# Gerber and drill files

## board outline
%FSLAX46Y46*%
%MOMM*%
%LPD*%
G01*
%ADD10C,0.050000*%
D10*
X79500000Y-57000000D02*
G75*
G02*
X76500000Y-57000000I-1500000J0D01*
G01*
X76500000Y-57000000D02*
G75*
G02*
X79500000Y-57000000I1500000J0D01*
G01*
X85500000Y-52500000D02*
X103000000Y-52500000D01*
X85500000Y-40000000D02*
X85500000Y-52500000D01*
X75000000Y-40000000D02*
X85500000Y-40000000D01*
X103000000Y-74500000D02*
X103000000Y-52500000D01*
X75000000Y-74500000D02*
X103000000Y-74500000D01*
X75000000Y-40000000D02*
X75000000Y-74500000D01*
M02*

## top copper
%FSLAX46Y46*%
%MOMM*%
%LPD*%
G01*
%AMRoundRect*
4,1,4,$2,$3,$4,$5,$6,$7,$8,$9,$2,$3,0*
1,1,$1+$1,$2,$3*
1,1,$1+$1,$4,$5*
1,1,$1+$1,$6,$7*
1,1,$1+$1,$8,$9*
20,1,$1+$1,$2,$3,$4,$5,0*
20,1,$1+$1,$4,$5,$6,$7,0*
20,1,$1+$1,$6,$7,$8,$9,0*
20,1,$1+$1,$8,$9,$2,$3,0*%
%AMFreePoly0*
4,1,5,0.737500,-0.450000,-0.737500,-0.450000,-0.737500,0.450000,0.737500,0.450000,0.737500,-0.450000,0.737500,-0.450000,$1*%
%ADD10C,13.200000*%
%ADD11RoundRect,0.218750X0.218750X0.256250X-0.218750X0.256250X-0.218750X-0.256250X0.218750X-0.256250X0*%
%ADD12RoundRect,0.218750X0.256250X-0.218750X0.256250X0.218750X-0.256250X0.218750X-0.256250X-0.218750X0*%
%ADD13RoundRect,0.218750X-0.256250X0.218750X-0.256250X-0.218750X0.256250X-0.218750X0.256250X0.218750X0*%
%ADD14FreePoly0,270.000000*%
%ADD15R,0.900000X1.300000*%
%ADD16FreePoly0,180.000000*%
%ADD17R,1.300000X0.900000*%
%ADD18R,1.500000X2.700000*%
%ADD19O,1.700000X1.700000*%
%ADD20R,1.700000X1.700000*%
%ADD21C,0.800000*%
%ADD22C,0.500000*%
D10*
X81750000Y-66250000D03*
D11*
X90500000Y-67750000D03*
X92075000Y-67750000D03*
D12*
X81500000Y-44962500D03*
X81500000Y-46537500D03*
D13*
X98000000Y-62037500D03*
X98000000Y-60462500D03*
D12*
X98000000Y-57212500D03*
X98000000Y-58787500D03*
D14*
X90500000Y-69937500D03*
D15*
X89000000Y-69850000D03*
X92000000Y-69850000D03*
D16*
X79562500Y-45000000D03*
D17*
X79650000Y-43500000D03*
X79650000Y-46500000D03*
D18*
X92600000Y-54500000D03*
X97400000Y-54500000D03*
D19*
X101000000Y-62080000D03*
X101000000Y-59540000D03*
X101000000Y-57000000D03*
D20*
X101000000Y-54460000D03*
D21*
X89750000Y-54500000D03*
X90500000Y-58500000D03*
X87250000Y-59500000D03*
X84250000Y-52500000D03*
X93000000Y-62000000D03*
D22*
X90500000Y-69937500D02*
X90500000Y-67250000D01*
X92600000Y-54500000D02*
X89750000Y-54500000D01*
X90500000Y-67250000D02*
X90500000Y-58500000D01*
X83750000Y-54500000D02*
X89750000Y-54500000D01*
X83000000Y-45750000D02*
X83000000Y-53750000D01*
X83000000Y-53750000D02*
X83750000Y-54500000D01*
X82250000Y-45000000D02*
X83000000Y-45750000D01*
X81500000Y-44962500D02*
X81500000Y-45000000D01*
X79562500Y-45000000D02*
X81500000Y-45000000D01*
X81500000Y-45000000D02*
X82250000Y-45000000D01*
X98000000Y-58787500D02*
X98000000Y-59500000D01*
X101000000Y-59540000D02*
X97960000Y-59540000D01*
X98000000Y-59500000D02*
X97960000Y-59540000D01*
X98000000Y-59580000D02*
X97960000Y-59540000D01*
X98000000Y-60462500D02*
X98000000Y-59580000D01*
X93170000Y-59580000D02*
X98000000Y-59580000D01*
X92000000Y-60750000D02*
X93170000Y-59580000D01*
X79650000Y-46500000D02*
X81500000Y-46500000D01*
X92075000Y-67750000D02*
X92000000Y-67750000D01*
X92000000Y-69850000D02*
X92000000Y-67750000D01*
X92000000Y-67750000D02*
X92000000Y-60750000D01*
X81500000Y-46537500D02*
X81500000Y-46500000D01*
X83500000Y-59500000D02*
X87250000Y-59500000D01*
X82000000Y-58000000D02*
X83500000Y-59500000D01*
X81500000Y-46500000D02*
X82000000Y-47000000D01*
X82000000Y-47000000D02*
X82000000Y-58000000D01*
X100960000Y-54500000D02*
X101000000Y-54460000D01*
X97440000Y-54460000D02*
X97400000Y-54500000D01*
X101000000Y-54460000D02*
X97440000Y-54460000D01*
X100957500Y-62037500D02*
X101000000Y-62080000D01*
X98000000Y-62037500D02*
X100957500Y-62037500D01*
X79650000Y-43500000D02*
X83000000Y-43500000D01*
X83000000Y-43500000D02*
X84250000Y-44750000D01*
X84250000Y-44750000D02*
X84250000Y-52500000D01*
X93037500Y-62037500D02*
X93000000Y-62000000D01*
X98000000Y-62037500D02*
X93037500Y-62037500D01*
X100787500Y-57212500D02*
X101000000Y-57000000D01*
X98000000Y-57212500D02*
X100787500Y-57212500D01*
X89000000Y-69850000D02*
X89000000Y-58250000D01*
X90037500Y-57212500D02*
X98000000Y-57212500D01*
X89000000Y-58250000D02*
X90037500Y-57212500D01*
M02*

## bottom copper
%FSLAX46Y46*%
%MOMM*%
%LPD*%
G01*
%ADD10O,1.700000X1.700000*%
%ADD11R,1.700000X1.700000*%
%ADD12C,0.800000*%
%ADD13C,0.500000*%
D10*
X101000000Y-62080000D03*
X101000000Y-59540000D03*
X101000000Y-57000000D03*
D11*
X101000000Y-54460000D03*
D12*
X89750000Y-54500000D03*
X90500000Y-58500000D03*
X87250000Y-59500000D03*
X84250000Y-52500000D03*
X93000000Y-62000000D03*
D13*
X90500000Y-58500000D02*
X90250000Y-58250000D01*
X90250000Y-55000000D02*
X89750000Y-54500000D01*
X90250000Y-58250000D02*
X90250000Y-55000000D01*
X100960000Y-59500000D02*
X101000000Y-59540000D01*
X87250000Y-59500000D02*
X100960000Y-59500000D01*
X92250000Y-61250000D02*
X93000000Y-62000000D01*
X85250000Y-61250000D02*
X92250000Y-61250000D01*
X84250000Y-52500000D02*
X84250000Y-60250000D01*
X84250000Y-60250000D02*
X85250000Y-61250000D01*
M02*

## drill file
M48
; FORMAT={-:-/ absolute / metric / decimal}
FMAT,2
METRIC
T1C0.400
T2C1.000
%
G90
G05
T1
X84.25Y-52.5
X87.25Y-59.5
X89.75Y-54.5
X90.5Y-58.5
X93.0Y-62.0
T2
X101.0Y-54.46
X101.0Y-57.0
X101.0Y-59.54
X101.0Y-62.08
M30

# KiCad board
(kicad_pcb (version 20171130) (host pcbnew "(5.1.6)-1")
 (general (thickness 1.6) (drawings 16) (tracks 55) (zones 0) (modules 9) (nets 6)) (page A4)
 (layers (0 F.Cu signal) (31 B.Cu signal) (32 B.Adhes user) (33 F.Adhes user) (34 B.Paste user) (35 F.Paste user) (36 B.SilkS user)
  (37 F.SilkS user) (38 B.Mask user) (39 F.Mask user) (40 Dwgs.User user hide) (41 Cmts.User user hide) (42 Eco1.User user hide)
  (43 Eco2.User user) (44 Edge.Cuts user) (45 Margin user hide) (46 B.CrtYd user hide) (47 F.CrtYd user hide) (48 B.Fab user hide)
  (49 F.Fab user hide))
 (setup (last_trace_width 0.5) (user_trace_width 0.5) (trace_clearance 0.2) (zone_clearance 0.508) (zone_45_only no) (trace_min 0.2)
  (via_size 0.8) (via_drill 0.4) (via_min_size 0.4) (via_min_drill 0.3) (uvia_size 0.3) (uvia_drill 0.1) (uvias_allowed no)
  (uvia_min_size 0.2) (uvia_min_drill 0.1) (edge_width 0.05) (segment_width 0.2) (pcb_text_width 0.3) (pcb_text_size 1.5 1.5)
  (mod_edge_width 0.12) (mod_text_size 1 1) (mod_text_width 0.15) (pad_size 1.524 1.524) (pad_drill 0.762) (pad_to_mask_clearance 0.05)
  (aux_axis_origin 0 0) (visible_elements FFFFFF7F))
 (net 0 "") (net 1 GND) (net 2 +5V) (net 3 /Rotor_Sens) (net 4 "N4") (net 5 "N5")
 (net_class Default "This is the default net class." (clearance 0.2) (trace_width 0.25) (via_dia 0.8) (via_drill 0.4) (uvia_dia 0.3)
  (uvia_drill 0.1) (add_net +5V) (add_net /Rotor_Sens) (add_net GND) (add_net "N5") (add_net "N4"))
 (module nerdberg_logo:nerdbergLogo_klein (layer F.Cu) (at 81.8 66.25)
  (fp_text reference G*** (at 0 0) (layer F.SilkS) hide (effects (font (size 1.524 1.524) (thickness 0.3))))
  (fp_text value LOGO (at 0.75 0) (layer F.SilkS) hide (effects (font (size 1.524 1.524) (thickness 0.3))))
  (pad e1 smd circle (at -0.05 0) (size 13.2 13.2) (layers F.Cu)))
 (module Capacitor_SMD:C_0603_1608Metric (layer F.Cu) (at 91.2875 67.75 180)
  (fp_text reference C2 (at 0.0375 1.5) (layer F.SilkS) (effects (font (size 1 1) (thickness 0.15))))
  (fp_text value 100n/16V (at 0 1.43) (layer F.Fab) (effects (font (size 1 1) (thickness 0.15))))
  (pad 2 smd roundrect (at 0.7875 0 180) (size 0.875 0.95) (layers F.Cu F.Paste F.Mask) (roundrect_rratio 0.25) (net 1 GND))
  (pad 1 smd roundrect (at -0.7875 0 180) (size 0.875 0.95) (layers F.Cu F.Paste F.Mask) (roundrect_rratio 0.25) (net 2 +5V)))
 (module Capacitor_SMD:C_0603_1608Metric (layer F.Cu) (at 81.5 45.75 90)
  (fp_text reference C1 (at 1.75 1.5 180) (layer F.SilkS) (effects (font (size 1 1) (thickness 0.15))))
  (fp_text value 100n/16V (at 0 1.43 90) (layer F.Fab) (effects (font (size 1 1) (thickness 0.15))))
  (pad 2 smd roundrect (at 0.7875 0 90) (size 0.875 0.95) (layers F.Cu F.Paste F.Mask) (roundrect_rratio 0.25) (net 1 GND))
  (pad 1 smd roundrect (at -0.7875 0 90) (size 0.875 0.95) (layers F.Cu F.Paste F.Mask) (roundrect_rratio 0.25) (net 2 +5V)))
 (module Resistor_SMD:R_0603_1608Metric (layer F.Cu) (at 98 61.25 270)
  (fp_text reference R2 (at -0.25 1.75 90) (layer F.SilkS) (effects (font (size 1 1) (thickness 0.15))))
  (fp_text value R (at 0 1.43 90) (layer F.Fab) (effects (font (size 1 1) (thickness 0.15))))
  (pad 2 smd roundrect (at 0.7875 0 270) (size 0.875 0.95) (layers F.Cu F.Paste F.Mask) (roundrect_rratio 0.25) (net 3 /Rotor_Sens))
  (pad 1 smd roundrect (at -0.7875 0 270) (size 0.875 0.95) (layers F.Cu F.Paste F.Mask) (roundrect_rratio 0.25) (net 2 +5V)))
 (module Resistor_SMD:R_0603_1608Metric (layer F.Cu) (at 98 58 90)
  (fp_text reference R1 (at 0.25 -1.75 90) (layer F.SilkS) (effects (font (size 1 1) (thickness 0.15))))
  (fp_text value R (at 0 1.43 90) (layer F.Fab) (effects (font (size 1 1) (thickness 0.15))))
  (pad 2 smd roundrect (at 0.7875 0 90) (size 0.875 0.95) (layers F.Cu F.Paste F.Mask) (roundrect_rratio 0.25) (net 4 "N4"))
  (pad 1 smd roundrect (at -0.7875 0 90) (size 0.875 0.95) (layers F.Cu F.Paste F.Mask) (roundrect_rratio 0.25) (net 2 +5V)))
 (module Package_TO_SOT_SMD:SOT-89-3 (layer F.Cu) (at 90.5 71.5 270)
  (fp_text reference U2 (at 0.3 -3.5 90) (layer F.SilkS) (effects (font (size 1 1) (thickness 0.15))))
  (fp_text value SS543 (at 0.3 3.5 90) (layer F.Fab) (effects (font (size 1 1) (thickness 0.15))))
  (pad 2 smd custom (at -1.5625 0 270) (size 1.475 0.9) (layers F.Cu F.Paste F.Mask) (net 1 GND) (zone_connect 2)
   (options (clearance outline) (anchor rect)) (primitives))
  (pad 3 smd rect (at -1.65 1.5 270) (size 1.3 0.9) (layers F.Cu F.Paste F.Mask) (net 4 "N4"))
  (pad 1 smd rect (at -1.65 -1.5 270) (size 1.3 0.9) (layers F.Cu F.Paste F.Mask) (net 2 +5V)))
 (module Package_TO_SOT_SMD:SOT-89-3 (layer F.Cu) (at 78 45 180)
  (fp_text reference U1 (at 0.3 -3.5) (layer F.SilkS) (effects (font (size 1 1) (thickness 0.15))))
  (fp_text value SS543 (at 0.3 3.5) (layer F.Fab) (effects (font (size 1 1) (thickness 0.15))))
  (pad 2 smd custom (at -1.5625 0 180) (size 1.475 0.9) (layers F.Cu F.Paste F.Mask) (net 1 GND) (zone_connect 2)
   (options (clearance outline) (anchor rect)) (primitives))
  (pad 3 smd rect (at -1.65 1.5 180) (size 1.3 0.9) (layers F.Cu F.Paste F.Mask) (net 3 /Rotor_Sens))
  (pad 1 smd rect (at -1.65 -1.5 180) (size 1.3 0.9) (layers F.Cu F.Paste F.Mask) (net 2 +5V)))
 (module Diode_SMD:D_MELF (layer F.Cu) (at 95 54.5 180)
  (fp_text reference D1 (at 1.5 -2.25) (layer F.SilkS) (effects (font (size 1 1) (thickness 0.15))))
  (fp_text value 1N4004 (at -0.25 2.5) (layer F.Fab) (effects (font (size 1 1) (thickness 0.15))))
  (pad 2 smd rect (at 2.4 0 180) (size 1.5 2.7) (layers F.Cu F.Paste F.Mask) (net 1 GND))
  (pad 1 smd rect (at -2.4 0 180) (size 1.5 2.7) (layers F.Cu F.Paste F.Mask) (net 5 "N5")))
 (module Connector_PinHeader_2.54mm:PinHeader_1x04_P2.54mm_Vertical (layer F.Cu) (at 101 54.46)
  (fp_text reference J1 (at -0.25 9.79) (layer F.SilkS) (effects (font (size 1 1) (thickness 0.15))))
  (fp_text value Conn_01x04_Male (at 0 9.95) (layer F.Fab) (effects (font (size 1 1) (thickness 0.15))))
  (pad 4 thru_hole oval (at 0 7.62) (size 1.7 1.7) (drill 1) (layers *.Cu *.Mask) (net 3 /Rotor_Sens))
  (pad 3 thru_hole oval (at 0 5.08) (size 1.7 1.7) (drill 1) (layers *.Cu *.Mask) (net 2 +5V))
  (pad 2 thru_hole oval (at 0 2.54) (size 1.7 1.7) (drill 1) (layers *.Cu *.Mask) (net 4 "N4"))
  (pad 1 thru_hole rect (at 0 0) (size 1.7 1.7) (drill 1) (layers *.Cu *.Mask) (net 5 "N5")))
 (gr_circle (center 78 57) (end 79.5 57) (layer Edge.Cuts) (width 0.05))
 (gr_line (start 85.5 52.5) (end 103 52.5) (layer Edge.Cuts) (width 0.05))
 (gr_line (start 85.5 40) (end 85.5 52.5) (layer Edge.Cuts) (width 0.05))
 (gr_line (start 75 40) (end 85.5 40) (layer Edge.Cuts) (width 0.05))
 (gr_line (start 103 74.5) (end 103 52.5) (layer Edge.Cuts) (width 0.05))
 (gr_line (start 75 74.5) (end 103 74.5) (layer Edge.Cuts) (width 0.05))
 (gr_line (start 75 40) (end 75 74.5) (layer Edge.Cuts) (width 0.05))
 (segment (start 90.5 69.9375) (end 90.5 67.25) (width 0.5) (layer F.Cu) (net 1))
 (via (at 89.75 54.5) (size 0.8) (drill 0.4) (layers F.Cu B.Cu) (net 1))
 (segment (start 92.6 54.5) (end 89.75 54.5) (width 0.5) (layer F.Cu) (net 1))
 (segment (start 90.5 67.25) (end 90.5 58.5) (width 0.5) (layer F.Cu) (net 1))
 (via (at 90.5 58.5) (size 0.8) (drill 0.4) (layers F.Cu B.Cu) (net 1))
 (segment (start 83.75 54.5) (end 89.75 54.5) (width 0.5) (layer F.Cu) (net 1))
 (segment (start 83 45.75) (end 83 53.75) (width 0.5) (layer F.Cu) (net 1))
 (segment (start 83 53.75) (end 83.75 54.5) (width 0.5) (layer F.Cu) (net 1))
 (segment (start 82.25 45) (end 83 45.75) (width 0.5) (layer F.Cu) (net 1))
 (segment (start 90.5 58.5) (end 90.25 58.25) (width 0.5) (layer B.Cu) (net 1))
 (segment (start 90.25 55) (end 89.75 54.5) (width 0.5) (layer B.Cu) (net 1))
 (segment (start 90.25 58.25) (end 90.25 55) (width 0.5) (layer B.Cu) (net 1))
 (segment (start 81.5 44.9625) (end 81.5 45) (width 0.5) (layer F.Cu) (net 1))
 (segment (start 79.5625 45) (end 81.5 45) (width 0.5) (layer F.Cu) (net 1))
 (segment (start 81.5 45) (end 82.25 45) (width 0.5) (layer F.Cu) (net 1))
 (segment (start 98 58.7875) (end 98 59.5) (width 0.5) (layer F.Cu) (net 2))
 (segment (start 101 59.54) (end 97.96 59.54) (width 0.5) (layer F.Cu) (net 2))
 (segment (start 98 59.5) (end 97.96 59.54) (width 0.5) (layer F.Cu) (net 2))
 (segment (start 98 59.58) (end 97.96 59.54) (width 0.5) (layer F.Cu) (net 2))
 (segment (start 98 60.4625) (end 98 59.58) (width 0.5) (layer F.Cu) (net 2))
 (via (at 87.25 59.5) (size 0.8) (drill 0.4) (layers F.Cu B.Cu) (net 2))
 (segment (start 100.96 59.5) (end 101 59.54) (width 0.5) (layer B.Cu) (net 2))
 (segment (start 87.25 59.5) (end 100.96 59.5) (width 0.5) (layer B.Cu) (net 2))
 (segment (start 93.17 59.58) (end 98 59.58) (width 0.5) (layer F.Cu) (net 2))
 (segment (start 92 60.75) (end 93.17 59.58) (width 0.5) (layer F.Cu) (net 2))
 (segment (start 79.65 46.5) (end 81.5 46.5) (width 0.5) (layer F.Cu) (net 2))
 (segment (start 92.075 67.75) (end 92 67.75) (width 0.5) (layer F.Cu) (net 2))
 (segment (start 92 69.85) (end 92 67.75) (width 0.5) (layer F.Cu) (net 2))
 (segment (start 92 67.75) (end 92 60.75) (width 0.5) (layer F.Cu) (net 2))
 (segment (start 81.5 46.5375) (end 81.5 46.5) (width 0.5) (layer F.Cu) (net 2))
 (segment (start 83.5 59.5) (end 87.25 59.5) (width 0.5) (layer F.Cu) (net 2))
 (segment (start 82 58) (end 83.5 59.5) (width 0.5) (layer F.Cu) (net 2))
 (segment (start 81.5 46.5) (end 82 47) (width 0.5) (layer F.Cu) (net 2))
 (segment (start 82 47) (end 82 58) (width 0.5) (layer F.Cu) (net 2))
 (segment (start 100.96 54.5) (end 101 54.46) (width 0.5) (layer F.Cu) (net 5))
 (segment (start 97.44 54.46) (end 97.4 54.5) (width 0.5) (layer F.Cu) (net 5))
 (segment (start 101 54.46) (end 97.44 54.46) (width 0.5) (layer F.Cu) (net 5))
 (segment (start 100.9575 62.0375) (end 101 62.08) (width 0.5) (layer F.Cu) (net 3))
 (segment (start 98 62.0375) (end 100.9575 62.0375) (width 0.5) (layer F.Cu) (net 3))
 (segment (start 79.65 43.5) (end 83 43.5) (width 0.5) (layer F.Cu) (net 3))
 (segment (start 83 43.5) (end 84.25 44.75) (width 0.5) (layer F.Cu) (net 3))
 (via (at 84.25 52.5) (size 0.8) (drill 0.4) (layers F.Cu B.Cu) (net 3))
 (segment (start 84.25 44.75) (end 84.25 52.5) (width 0.5) (layer F.Cu) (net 3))
 (via (at 93 62) (size 0.8) (drill 0.4) (layers F.Cu B.Cu) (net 3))
 (segment (start 93.0375 62.0375) (end 93 62) (width 0.5) (layer F.Cu) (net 3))
 (segment (start 98 62.0375) (end 93.0375 62.0375) (width 0.5) (layer F.Cu) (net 3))
 (segment (start 92.25 61.25) (end 93 62) (width 0.5) (layer B.Cu) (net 3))
 (segment (start 85.25 61.25) (end 92.25 61.25) (width 0.5) (layer B.Cu) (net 3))
 (segment (start 84.25 52.5) (end 84.25 60.25) (width 0.5) (layer B.Cu) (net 3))
 (segment (start 84.25 60.25) (end 85.25 61.25) (width 0.5) (layer B.Cu) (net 3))
 (segment (start 100.7875 57.2125) (end 101 57) (width 0.5) (layer F.Cu) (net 4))
 (segment (start 98 57.2125) (end 100.7875 57.2125) (width 0.5) (layer F.Cu) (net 4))
 (segment (start 89 69.85) (end 89 58.25) (width 0.5) (layer F.Cu) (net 4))
 (segment (start 90.0375 57.2125) (end 98 57.2125) (width 0.5) (layer F.Cu) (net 4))
 (segment (start 89 58.25) (end 90.0375 57.2125) (width 0.5) (layer F.Cu) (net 4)))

